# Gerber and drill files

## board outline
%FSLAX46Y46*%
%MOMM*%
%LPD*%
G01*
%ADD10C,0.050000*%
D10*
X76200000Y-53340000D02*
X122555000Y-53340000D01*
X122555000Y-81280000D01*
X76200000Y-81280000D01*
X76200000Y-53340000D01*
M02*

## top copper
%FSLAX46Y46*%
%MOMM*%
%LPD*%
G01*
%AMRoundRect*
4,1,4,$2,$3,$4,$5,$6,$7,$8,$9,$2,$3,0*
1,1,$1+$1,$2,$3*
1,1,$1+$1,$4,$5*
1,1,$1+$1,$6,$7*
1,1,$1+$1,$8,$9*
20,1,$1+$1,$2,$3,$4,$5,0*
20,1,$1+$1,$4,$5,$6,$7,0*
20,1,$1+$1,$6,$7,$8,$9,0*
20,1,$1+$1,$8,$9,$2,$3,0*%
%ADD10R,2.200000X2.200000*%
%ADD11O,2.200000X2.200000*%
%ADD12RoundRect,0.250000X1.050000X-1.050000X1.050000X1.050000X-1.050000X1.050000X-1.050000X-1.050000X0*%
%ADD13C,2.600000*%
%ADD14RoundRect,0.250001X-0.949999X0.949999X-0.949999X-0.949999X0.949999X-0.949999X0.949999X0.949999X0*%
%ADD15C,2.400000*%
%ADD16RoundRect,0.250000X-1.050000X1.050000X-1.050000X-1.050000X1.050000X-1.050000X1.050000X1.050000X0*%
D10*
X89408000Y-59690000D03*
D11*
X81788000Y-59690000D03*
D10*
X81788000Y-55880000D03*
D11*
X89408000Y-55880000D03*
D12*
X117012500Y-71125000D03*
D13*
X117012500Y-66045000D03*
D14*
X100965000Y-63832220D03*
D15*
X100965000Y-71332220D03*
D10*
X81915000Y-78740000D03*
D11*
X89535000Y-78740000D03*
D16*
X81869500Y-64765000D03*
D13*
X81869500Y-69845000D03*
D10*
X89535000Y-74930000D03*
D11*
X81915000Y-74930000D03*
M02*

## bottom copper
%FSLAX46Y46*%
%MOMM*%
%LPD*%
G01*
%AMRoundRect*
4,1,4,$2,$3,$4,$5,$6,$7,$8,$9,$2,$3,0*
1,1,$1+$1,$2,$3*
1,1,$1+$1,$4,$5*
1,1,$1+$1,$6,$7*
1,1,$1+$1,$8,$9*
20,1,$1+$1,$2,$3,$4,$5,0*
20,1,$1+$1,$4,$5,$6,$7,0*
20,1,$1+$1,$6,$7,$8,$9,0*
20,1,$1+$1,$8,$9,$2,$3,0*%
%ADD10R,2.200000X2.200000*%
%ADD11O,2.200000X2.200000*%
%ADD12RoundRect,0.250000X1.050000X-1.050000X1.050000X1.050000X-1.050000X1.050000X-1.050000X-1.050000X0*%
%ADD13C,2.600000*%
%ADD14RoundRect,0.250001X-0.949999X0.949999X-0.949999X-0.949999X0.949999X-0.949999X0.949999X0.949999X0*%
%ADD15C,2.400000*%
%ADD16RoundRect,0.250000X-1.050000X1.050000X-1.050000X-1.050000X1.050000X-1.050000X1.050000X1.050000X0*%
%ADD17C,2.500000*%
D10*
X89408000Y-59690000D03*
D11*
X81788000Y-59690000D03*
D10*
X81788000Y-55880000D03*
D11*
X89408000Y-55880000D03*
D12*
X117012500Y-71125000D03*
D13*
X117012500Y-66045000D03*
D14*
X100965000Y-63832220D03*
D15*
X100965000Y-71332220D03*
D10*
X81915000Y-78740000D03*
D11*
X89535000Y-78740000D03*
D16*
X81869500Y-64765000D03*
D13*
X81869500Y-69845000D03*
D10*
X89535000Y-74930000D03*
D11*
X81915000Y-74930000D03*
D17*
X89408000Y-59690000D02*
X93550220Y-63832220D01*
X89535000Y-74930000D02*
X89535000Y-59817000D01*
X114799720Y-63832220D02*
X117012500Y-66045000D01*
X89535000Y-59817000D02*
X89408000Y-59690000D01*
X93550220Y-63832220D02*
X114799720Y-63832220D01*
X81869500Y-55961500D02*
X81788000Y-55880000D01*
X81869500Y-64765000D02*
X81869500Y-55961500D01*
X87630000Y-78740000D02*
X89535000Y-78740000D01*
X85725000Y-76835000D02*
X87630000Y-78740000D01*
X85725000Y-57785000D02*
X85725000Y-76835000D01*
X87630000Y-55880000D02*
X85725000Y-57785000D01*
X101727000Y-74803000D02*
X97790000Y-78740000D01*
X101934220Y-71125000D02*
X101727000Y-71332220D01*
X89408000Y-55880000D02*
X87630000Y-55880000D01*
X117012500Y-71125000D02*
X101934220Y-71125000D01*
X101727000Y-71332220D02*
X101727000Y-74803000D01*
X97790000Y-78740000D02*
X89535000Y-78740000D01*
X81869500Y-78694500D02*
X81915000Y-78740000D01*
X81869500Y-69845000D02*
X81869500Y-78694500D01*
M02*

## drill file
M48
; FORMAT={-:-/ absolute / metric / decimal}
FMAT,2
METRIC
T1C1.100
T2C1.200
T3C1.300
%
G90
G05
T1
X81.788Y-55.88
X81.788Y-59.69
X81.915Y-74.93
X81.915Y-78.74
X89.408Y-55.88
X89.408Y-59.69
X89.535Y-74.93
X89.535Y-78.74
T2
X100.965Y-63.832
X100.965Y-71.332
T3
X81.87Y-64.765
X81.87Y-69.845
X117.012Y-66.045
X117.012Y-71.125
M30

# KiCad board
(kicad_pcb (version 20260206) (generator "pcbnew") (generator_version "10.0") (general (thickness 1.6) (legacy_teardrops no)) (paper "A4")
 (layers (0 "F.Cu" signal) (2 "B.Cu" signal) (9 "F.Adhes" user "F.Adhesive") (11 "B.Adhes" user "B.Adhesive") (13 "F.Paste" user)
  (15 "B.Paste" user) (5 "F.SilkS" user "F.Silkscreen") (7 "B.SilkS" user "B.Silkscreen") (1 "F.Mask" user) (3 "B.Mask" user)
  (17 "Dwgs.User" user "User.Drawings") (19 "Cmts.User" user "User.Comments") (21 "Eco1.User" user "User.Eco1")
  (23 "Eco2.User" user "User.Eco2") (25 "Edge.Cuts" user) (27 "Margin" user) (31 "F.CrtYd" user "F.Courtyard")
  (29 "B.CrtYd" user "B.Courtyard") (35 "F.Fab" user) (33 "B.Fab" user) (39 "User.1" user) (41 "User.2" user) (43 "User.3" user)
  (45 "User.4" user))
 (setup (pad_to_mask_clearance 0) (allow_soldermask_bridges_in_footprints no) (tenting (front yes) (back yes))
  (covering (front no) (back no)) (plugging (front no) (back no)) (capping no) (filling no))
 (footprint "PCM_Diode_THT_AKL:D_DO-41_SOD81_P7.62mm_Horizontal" (layer "F.Cu") (at 89.408 59.69 180)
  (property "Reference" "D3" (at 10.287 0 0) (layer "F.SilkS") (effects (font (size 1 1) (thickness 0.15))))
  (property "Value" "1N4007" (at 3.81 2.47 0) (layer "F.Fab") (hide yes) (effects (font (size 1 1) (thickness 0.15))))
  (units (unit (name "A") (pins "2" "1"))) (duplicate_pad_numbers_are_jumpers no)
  (pad "1" thru_hole rect (at 0 0 180) (size 2.2 2.2) (drill 1.1) (layers "*.Cu" "*.Mask") (remove_unused_layers no) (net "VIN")
   (teardrops (best_length_ratio 0.5) (max_length 1) (best_width_ratio 1) (max_width 2) (curved_edges no) (filter_ratio 0.9) (enabled yes)
    (allow_two_segments yes) (prefer_zone_connections yes)))
  (pad "2" thru_hole oval (at 7.62 0 180) (size 2.2 2.2) (drill 1.1) (layers "*.Cu" "*.Mask") (remove_unused_layers no) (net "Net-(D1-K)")
   (teardrops (best_length_ratio 0.5) (max_length 1) (best_width_ratio 1) (max_width 2) (curved_edges no) (filter_ratio 0.9) (enabled yes)
    (allow_two_segments yes) (prefer_zone_connections yes))))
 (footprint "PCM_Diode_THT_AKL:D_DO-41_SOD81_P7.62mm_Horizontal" (layer "F.Cu") (at 81.788 55.88)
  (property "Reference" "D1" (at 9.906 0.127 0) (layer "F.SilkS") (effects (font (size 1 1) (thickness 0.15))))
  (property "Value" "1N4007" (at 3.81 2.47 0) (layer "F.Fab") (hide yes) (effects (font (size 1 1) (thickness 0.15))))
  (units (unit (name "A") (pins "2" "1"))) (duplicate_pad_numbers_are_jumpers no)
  (pad "1" thru_hole rect (at 0 0) (size 2.2 2.2) (drill 1.1) (layers "*.Cu" "*.Mask") (remove_unused_layers no) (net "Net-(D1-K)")
   (teardrops (best_length_ratio 0.5) (max_length 1) (best_width_ratio 1) (max_width 2) (curved_edges no) (filter_ratio 0.9) (enabled yes)
    (allow_two_segments yes) (prefer_zone_connections yes)))
  (pad "2" thru_hole oval (at 7.62 0) (size 2.2 2.2) (drill 1.1) (layers "*.Cu" "*.Mask") (remove_unused_layers no) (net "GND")
   (teardrops (best_length_ratio 0.5) (max_length 1) (best_width_ratio 1) (max_width 2) (curved_edges no) (filter_ratio 0.9) (enabled yes)
    (allow_two_segments yes) (prefer_zone_connections yes))))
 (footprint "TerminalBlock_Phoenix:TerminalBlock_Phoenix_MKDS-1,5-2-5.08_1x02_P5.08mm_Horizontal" (layer "F.Cu") (at 117.0125 71.125 90)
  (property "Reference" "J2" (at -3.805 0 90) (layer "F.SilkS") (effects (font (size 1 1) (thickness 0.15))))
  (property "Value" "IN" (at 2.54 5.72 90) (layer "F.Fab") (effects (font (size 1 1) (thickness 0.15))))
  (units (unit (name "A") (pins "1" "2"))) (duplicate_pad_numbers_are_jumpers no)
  (pad "1" thru_hole roundrect (at 0 0 90) (size 2.6 2.6) (drill 1.3) (layers "*.Cu" "*.Mask") (remove_unused_layers no)
   (roundrect_rratio 0.096154) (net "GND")
   (teardrops (best_length_ratio 0.5) (max_length 1) (best_width_ratio 1) (max_width 2) (curved_edges no) (filter_ratio 0.9) (enabled yes)
    (allow_two_segments yes) (prefer_zone_connections yes)))
  (pad "2" thru_hole circle (at 5.08 0 90) (size 2.6 2.6) (drill 1.3) (layers "*.Cu" "*.Mask") (remove_unused_layers no) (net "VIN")
   (teardrops (best_length_ratio 0.5) (max_length 1) (best_width_ratio 1) (max_width 2) (curved_edges no) (filter_ratio 0.9) (enabled yes)
    (allow_two_segments yes) (prefer_zone_connections yes))))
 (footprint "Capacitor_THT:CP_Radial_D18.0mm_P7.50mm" (layer "F.Cu") (at 100.965 63.83222 -90)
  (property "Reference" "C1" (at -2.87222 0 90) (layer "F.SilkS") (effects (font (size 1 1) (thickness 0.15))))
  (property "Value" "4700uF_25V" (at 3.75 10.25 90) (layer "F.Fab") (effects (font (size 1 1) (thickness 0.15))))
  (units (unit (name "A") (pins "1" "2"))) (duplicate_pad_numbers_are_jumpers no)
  (pad "1" thru_hole roundrect (at 0 0 270) (size 2.4 2.4) (drill 1.2) (layers "*.Cu" "*.Mask") (remove_unused_layers no)
   (roundrect_rratio 0.104167) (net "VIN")
   (teardrops (best_length_ratio 0.5) (max_length 1) (best_width_ratio 1) (max_width 2) (curved_edges no) (filter_ratio 0.9) (enabled yes)
    (allow_two_segments yes) (prefer_zone_connections yes)))
  (pad "2" thru_hole circle (at 7.5 0 270) (size 2.4 2.4) (drill 1.2) (layers "*.Cu" "*.Mask") (remove_unused_layers no) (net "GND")
   (teardrops (best_length_ratio 0.5) (max_length 1) (best_width_ratio 1) (max_width 2) (curved_edges no) (filter_ratio 0.9) (enabled yes)
    (allow_two_segments yes) (prefer_zone_connections yes))))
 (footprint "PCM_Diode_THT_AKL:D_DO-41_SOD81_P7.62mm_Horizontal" (layer "F.Cu") (at 81.915 78.74)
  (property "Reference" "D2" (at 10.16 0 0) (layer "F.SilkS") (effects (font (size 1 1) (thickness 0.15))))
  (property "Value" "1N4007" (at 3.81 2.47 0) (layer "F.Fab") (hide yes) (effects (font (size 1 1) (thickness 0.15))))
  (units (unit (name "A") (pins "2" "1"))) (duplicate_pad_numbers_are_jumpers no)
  (pad "1" thru_hole rect (at 0 0) (size 2.2 2.2) (drill 1.1) (layers "*.Cu" "*.Mask") (remove_unused_layers no) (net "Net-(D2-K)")
   (teardrops (best_length_ratio 0.5) (max_length 1) (best_width_ratio 1) (max_width 2) (curved_edges no) (filter_ratio 0.9) (enabled yes)
    (allow_two_segments yes) (prefer_zone_connections yes)))
  (pad "2" thru_hole oval (at 7.62 0) (size 2.2 2.2) (drill 1.1) (layers "*.Cu" "*.Mask") (remove_unused_layers no) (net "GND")
   (teardrops (best_length_ratio 0.5) (max_length 1) (best_width_ratio 1) (max_width 2) (curved_edges no) (filter_ratio 0.9) (enabled yes)
    (allow_two_segments yes) (prefer_zone_connections yes))))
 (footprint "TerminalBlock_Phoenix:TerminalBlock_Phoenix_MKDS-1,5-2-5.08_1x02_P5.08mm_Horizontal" (layer "F.Cu") (at 81.8695 64.765 -90)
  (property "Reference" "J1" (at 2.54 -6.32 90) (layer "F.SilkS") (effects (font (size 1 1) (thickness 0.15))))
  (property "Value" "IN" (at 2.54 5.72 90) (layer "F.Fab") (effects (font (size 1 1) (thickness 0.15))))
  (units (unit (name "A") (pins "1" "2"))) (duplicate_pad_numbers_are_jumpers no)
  (pad "1" thru_hole roundrect (at 0 0 270) (size 2.6 2.6) (drill 1.3) (layers "*.Cu" "*.Mask") (remove_unused_layers no)
   (roundrect_rratio 0.096154) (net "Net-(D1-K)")
   (teardrops (best_length_ratio 0.5) (max_length 1) (best_width_ratio 1) (max_width 2) (curved_edges no) (filter_ratio 0.9) (enabled yes)
    (allow_two_segments yes) (prefer_zone_connections yes)))
  (pad "2" thru_hole circle (at 5.08 0 270) (size 2.6 2.6) (drill 1.3) (layers "*.Cu" "*.Mask") (remove_unused_layers no) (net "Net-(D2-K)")
   (teardrops (best_length_ratio 0.5) (max_length 1) (best_width_ratio 1) (max_width 2) (curved_edges no) (filter_ratio 0.9) (enabled yes)
    (allow_two_segments yes) (prefer_zone_connections yes))))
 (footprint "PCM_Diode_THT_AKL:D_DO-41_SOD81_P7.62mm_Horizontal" (layer "F.Cu") (at 89.535 74.93 180)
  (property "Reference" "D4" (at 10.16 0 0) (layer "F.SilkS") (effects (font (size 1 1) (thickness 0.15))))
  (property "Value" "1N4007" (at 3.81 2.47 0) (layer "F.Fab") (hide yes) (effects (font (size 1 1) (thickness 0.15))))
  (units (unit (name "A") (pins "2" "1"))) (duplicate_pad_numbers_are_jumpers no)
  (pad "1" thru_hole rect (at 0 0 180) (size 2.2 2.2) (drill 1.1) (layers "*.Cu" "*.Mask") (remove_unused_layers no) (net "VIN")
   (teardrops (best_length_ratio 0.5) (max_length 1) (best_width_ratio 1) (max_width 2) (curved_edges no) (filter_ratio 0.9) (enabled yes)
    (allow_two_segments yes) (prefer_zone_connections yes)))
  (pad "2" thru_hole oval (at 7.62 0 180) (size 2.2 2.2) (drill 1.1) (layers "*.Cu" "*.Mask") (remove_unused_layers no) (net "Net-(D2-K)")
   (teardrops (best_length_ratio 0.5) (max_length 1) (best_width_ratio 1) (max_width 2) (curved_edges no) (filter_ratio 0.9) (enabled yes)
    (allow_two_segments yes) (prefer_zone_connections yes))))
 (gr_rect (start 76.2 53.34) (end 122.555 81.28) (stroke (width 0.05) (type default)) (fill no) (layer "Edge.Cuts"))
 (segment (start 89.408 59.69) (end 93.55022 63.83222) (width 2.5) (layer "B.Cu") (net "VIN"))
 (segment (start 89.535 74.93) (end 89.535 59.817) (width 2.5) (layer "B.Cu") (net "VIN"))
 (segment (start 114.79972 63.83222) (end 117.0125 66.045) (width 2.5) (layer "B.Cu") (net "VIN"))
 (segment (start 89.535 59.817) (end 89.408 59.69) (width 2.5) (layer "B.Cu") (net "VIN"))
 (segment (start 93.55022 63.83222) (end 114.79972 63.83222) (width 2.5) (layer "B.Cu") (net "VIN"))
 (segment (start 81.8695 55.9615) (end 81.788 55.88) (width 2.5) (layer "B.Cu") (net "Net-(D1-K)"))
 (segment (start 81.8695 64.765) (end 81.8695 55.9615) (width 2.5) (layer "B.Cu") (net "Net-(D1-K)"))
 (segment (start 87.63 78.74) (end 89.535 78.74) (width 2.5) (layer "B.Cu") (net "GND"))
 (segment (start 85.725 76.835) (end 87.63 78.74) (width 2.5) (layer "B.Cu") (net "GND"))
 (segment (start 85.725 57.785) (end 85.725 76.835) (width 2.5) (layer "B.Cu") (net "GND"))
 (segment (start 87.63 55.88) (end 85.725 57.785) (width 2.5) (layer "B.Cu") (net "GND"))
 (segment (start 101.727 74.803) (end 97.79 78.74) (width 2.5) (layer "B.Cu") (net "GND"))
 (segment (start 101.93422 71.125) (end 101.727 71.33222) (width 2.5) (layer "B.Cu") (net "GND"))
 (segment (start 89.408 55.88) (end 87.63 55.88) (width 2.5) (layer "B.Cu") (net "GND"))
 (segment (start 117.0125 71.125) (end 101.93422 71.125) (width 2.5) (layer "B.Cu") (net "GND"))
 (segment (start 101.727 71.33222) (end 101.727 74.803) (width 2.5) (layer "B.Cu") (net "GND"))
 (segment (start 97.79 78.74) (end 89.535 78.74) (width 2.5) (layer "B.Cu") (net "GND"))
 (segment (start 81.8695 78.6945) (end 81.915 78.74) (width 2.5) (layer "B.Cu") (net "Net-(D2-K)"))
 (segment (start 81.8695 69.845) (end 81.8695 78.6945) (width 2.5) (layer "B.Cu") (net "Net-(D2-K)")))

